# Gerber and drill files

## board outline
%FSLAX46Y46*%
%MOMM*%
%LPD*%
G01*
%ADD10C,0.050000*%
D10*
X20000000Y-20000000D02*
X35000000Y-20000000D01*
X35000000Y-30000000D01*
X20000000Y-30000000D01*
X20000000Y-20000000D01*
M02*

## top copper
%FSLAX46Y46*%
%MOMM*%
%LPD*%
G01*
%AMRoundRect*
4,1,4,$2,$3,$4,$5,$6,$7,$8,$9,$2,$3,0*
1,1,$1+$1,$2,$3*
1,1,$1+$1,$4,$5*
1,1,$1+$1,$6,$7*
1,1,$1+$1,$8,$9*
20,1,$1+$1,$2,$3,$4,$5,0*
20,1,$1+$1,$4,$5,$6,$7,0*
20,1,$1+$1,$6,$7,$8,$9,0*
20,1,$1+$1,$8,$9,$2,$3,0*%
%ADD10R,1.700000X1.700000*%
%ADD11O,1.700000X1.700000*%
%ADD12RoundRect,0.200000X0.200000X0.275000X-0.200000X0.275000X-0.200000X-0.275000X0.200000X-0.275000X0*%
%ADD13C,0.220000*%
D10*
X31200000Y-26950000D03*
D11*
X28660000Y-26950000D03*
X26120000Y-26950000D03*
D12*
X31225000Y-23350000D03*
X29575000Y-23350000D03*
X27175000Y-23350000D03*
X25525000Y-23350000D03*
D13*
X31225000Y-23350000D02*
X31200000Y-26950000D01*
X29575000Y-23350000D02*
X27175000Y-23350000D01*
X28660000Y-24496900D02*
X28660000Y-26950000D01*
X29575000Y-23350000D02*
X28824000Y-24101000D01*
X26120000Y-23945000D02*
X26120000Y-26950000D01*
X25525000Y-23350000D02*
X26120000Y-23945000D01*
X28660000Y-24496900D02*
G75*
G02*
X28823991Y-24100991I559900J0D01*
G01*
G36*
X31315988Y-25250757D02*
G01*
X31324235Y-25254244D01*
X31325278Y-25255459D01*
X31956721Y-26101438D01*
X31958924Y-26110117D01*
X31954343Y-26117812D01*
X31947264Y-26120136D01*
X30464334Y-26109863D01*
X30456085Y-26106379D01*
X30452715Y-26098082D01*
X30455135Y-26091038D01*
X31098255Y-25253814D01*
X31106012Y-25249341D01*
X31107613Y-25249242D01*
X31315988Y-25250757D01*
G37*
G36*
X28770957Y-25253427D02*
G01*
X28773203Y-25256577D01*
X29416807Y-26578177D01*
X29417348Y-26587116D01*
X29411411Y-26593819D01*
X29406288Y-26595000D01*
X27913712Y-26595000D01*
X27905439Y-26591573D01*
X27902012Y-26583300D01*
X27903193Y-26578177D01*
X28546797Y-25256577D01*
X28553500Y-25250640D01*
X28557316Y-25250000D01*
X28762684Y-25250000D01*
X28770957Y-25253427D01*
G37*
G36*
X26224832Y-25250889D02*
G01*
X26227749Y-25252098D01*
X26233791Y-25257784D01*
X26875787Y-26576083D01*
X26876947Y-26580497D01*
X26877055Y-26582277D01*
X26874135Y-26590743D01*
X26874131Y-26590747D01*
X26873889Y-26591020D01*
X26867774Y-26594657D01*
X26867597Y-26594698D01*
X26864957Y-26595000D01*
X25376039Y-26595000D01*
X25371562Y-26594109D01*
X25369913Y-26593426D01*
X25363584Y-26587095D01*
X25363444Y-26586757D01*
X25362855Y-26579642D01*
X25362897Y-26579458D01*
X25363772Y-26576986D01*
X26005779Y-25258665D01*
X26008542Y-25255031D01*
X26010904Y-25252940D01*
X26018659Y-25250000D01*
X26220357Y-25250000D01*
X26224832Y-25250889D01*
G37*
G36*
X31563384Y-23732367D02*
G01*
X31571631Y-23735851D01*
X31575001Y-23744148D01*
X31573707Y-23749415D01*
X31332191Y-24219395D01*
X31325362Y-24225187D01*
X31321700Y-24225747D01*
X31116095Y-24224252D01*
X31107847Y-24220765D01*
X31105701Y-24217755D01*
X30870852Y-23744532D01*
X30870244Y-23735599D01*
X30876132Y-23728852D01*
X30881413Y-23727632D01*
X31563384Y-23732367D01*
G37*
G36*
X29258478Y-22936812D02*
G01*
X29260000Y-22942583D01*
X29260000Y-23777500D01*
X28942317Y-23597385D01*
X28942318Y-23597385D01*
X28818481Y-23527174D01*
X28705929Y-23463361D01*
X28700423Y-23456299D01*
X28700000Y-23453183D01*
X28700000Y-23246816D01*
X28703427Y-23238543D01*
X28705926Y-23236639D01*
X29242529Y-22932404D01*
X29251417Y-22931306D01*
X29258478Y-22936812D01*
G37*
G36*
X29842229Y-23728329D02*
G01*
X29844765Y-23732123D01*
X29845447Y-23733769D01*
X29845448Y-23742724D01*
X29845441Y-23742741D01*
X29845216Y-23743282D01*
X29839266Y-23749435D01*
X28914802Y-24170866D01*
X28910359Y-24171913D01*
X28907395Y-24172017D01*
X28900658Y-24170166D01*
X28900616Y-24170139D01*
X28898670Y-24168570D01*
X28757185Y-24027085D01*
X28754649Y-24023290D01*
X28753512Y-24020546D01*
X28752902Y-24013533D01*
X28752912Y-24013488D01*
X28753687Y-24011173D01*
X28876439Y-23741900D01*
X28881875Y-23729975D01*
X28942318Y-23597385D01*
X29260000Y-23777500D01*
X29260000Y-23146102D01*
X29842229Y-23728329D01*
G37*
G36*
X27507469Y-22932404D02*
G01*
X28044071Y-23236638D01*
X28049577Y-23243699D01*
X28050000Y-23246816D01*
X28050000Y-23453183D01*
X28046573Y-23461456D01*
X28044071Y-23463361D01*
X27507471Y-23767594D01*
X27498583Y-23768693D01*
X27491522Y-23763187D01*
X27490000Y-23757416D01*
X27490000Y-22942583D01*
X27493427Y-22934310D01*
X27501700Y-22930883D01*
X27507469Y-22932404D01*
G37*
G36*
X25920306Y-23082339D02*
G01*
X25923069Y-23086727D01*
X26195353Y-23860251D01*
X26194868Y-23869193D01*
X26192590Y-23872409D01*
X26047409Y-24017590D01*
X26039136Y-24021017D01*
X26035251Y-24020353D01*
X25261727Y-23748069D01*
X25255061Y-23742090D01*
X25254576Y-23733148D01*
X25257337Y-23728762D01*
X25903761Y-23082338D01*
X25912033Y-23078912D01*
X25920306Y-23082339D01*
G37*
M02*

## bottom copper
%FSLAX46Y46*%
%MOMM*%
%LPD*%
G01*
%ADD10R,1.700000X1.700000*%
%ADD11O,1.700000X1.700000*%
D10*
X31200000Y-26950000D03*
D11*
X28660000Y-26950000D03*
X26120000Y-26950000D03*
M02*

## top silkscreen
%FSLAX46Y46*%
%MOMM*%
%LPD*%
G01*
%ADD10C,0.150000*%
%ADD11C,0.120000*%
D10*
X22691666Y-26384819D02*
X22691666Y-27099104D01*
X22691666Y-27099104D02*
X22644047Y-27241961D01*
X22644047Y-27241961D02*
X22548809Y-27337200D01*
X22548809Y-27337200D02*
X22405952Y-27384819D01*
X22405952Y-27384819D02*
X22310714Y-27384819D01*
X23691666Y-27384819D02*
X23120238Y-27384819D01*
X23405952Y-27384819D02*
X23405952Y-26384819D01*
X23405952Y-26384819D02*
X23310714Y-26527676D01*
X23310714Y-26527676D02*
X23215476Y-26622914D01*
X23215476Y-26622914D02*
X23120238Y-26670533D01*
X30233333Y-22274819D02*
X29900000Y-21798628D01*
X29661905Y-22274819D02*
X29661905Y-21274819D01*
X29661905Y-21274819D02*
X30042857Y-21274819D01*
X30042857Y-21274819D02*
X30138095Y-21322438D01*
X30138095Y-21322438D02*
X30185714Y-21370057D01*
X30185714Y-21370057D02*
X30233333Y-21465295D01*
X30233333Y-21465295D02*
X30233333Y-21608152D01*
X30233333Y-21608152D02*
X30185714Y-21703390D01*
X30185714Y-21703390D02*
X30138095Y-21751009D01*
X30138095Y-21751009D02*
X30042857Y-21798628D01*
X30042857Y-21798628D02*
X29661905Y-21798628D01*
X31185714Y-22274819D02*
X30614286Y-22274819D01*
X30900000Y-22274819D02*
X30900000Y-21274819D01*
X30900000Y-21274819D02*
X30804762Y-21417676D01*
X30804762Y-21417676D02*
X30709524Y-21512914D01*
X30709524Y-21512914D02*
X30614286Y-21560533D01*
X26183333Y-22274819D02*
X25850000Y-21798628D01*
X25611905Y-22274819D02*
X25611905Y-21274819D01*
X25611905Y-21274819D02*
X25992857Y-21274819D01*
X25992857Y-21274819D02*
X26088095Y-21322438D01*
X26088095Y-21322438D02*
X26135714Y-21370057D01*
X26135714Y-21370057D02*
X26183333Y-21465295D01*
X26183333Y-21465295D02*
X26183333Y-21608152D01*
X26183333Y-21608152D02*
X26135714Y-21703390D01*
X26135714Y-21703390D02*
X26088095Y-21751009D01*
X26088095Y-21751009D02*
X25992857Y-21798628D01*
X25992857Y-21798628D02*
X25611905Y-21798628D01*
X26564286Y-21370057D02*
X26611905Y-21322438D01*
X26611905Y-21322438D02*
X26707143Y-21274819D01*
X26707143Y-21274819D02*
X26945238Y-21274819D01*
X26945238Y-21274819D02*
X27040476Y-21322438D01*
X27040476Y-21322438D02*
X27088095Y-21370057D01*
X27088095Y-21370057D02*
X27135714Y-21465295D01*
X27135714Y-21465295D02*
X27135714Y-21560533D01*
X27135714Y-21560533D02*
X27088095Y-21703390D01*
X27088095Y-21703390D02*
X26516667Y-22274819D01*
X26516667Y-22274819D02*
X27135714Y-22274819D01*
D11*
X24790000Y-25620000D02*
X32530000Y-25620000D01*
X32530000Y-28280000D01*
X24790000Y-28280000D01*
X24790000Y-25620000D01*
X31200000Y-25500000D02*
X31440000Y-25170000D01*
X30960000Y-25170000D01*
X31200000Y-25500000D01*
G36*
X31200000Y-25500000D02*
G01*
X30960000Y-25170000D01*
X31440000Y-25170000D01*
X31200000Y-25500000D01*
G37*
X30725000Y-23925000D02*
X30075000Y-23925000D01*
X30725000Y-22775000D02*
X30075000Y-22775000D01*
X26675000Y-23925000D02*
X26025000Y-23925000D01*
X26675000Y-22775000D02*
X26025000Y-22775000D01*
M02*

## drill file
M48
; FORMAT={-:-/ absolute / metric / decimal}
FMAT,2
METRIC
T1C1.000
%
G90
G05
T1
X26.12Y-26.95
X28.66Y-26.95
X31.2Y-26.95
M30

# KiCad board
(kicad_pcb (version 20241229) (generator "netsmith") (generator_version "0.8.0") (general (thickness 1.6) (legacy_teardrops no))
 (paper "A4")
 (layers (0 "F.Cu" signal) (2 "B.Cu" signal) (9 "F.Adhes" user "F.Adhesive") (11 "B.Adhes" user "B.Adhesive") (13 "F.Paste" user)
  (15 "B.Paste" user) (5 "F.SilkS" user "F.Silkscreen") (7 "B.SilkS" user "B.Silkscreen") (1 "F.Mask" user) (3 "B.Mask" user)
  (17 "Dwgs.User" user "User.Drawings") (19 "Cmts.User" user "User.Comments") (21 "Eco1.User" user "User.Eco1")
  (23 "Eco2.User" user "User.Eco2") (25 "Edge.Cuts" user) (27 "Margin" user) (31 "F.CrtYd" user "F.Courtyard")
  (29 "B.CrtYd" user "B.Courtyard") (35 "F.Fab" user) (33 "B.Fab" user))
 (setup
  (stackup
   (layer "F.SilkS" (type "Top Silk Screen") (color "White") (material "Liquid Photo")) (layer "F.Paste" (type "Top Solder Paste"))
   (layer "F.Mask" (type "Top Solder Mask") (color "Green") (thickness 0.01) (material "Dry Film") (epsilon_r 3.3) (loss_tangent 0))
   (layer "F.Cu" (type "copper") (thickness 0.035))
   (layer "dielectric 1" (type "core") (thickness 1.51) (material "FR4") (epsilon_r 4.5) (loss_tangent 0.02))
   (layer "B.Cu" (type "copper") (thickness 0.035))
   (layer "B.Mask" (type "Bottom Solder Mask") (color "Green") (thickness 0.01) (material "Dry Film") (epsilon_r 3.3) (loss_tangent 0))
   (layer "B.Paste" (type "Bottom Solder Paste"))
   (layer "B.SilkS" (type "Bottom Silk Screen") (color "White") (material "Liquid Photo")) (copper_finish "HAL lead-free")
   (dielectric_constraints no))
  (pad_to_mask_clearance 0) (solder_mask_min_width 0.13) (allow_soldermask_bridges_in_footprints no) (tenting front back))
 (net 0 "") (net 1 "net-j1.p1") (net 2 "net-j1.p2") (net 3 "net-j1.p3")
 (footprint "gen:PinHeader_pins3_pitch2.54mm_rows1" (layer "F.Cu") (at 31.2 26.95 270)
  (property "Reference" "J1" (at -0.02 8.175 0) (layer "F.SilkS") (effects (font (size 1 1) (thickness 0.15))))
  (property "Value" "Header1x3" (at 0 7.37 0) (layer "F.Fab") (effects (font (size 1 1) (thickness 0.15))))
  (pad "1" thru_hole rect (at 0 0 270) (size 1.7 1.7) (drill 1) (layers "*.Cu" "*.Mask") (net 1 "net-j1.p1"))
  (pad "2" thru_hole oval (at 0 2.54 270) (size 1.7 1.7) (drill 1) (layers "*.Cu" "*.Mask") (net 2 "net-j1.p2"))
  (pad "3" thru_hole oval (at 0 5.08 270) (size 1.7 1.7) (drill 1) (layers "*.Cu" "*.Mask") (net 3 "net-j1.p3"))
  (fp_rect (start -1.33 -1.33) (end 1.33 6.41) (stroke (width 0.12) (type solid)) (fill no) (layer "F.SilkS"))
  (fp_poly (pts (xy -1.45 0) (xy -1.78 -0.24) (xy -1.78 0.24)) (stroke (width 0.12) (type solid)) (fill solid) (layer "F.SilkS")))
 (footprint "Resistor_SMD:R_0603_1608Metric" (layer "F.Cu") (at 30.4 23.35 180)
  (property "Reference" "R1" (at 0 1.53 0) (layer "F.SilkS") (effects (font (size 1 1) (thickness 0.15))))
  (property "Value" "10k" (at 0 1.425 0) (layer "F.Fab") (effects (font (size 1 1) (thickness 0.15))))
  (pad "1" smd roundrect (at -0.825 0 180) (size 0.8 0.95) (layers "F.Cu" "F.Mask" "F.Paste") (roundrect_rratio 0.25) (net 1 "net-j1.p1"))
  (pad "2" smd roundrect (at 0.825 0 180) (size 0.8 0.95) (layers "F.Cu" "F.Mask" "F.Paste") (roundrect_rratio 0.25) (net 2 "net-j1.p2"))
  (fp_line (start -0.325 -0.575) (end 0.325 -0.575) (stroke (width 0.12) (type solid)) (layer "F.SilkS"))
  (fp_line (start -0.325 0.575) (end 0.325 0.575) (stroke (width 0.12) (type solid)) (layer "F.SilkS")))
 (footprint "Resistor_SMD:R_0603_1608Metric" (layer "F.Cu") (at 26.35 23.35 180)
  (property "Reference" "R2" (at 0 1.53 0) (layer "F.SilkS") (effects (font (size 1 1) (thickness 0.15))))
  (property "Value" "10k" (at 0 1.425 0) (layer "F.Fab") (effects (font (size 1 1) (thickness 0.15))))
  (pad "1" smd roundrect (at -0.825 0 180) (size 0.8 0.95) (layers "F.Cu" "F.Mask" "F.Paste") (roundrect_rratio 0.25) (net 2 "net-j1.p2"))
  (pad "2" smd roundrect (at 0.825 0 180) (size 0.8 0.95) (layers "F.Cu" "F.Mask" "F.Paste") (roundrect_rratio 0.25) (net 3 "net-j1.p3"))
  (fp_line (start -0.325 -0.575) (end 0.325 -0.575) (stroke (width 0.12) (type solid)) (layer "F.SilkS"))
  (fp_line (start -0.325 0.575) (end 0.325 0.575) (stroke (width 0.12) (type solid)) (layer "F.SilkS")))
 (segment (start 31.225 23.35) (end 31.2 26.95) (width 0.22) (layer "F.Cu") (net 1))
 (segment (start 29.575 23.35) (end 27.175 23.35) (width 0.22) (layer "F.Cu") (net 2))
 (segment (start 28.66 24.4969) (end 28.66 26.95) (width 0.22) (layer "F.Cu") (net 2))
 (segment (start 29.575 23.35) (end 28.824 24.101) (width 0.22) (layer "F.Cu") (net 2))
 (segment (start 26.12 23.945) (end 26.12 26.95) (width 0.22) (layer "F.Cu") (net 3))
 (segment (start 25.525 23.35) (end 26.12 23.945) (width 0.22) (layer "F.Cu") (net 3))
 (arc (start 28.66 24.4969) (mid 28.7026 24.2827) (end 28.824 24.101) (width 0.22) (layer "F.Cu") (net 2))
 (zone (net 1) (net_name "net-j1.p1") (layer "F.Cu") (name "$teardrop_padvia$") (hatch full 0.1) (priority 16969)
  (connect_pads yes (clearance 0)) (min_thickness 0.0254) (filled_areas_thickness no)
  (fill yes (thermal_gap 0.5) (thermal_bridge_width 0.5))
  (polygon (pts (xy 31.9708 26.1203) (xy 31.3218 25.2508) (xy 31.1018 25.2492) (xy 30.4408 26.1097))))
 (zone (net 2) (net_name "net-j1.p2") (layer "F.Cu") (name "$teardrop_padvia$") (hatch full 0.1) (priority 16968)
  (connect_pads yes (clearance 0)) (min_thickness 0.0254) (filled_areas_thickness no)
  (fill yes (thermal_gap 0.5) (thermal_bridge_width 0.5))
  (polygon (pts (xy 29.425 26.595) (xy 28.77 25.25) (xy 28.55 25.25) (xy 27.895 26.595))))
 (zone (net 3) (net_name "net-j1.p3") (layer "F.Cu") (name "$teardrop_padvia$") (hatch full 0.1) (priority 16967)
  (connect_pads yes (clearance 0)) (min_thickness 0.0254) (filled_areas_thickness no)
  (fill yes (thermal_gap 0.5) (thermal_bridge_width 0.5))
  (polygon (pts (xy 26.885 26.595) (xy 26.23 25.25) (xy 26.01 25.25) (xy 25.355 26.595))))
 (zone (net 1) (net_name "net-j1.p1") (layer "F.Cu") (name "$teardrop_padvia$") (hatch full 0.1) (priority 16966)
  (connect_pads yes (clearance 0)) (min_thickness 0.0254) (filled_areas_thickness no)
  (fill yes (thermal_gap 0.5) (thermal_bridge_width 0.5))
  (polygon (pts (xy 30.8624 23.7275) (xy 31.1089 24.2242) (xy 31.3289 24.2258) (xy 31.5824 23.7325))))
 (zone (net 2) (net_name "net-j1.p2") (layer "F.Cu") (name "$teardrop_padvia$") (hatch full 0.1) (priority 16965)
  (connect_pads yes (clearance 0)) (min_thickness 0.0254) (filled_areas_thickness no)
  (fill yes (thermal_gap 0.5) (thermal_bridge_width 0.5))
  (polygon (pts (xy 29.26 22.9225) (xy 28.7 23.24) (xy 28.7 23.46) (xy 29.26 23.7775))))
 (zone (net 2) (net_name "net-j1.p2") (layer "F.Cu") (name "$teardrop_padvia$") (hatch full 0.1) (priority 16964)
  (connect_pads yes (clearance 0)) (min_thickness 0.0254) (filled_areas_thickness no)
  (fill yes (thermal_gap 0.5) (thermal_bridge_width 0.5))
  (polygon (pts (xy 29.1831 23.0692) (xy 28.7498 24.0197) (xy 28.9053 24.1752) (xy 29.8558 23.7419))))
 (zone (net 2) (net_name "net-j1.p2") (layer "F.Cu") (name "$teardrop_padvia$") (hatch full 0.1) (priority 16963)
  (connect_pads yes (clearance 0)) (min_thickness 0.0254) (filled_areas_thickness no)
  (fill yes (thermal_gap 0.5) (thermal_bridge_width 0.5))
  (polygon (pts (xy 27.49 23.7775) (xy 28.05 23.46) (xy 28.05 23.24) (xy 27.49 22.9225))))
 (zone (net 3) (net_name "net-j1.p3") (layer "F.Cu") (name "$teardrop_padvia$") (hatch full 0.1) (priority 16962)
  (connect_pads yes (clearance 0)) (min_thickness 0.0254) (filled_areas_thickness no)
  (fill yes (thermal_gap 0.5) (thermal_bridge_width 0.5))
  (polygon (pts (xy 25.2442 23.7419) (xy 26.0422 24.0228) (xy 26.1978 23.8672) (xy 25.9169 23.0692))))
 (gr_rect (start 20 20) (end 35 30) (stroke (width 0.05) (type default)) (fill no) (layer "Edge.Cuts")))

